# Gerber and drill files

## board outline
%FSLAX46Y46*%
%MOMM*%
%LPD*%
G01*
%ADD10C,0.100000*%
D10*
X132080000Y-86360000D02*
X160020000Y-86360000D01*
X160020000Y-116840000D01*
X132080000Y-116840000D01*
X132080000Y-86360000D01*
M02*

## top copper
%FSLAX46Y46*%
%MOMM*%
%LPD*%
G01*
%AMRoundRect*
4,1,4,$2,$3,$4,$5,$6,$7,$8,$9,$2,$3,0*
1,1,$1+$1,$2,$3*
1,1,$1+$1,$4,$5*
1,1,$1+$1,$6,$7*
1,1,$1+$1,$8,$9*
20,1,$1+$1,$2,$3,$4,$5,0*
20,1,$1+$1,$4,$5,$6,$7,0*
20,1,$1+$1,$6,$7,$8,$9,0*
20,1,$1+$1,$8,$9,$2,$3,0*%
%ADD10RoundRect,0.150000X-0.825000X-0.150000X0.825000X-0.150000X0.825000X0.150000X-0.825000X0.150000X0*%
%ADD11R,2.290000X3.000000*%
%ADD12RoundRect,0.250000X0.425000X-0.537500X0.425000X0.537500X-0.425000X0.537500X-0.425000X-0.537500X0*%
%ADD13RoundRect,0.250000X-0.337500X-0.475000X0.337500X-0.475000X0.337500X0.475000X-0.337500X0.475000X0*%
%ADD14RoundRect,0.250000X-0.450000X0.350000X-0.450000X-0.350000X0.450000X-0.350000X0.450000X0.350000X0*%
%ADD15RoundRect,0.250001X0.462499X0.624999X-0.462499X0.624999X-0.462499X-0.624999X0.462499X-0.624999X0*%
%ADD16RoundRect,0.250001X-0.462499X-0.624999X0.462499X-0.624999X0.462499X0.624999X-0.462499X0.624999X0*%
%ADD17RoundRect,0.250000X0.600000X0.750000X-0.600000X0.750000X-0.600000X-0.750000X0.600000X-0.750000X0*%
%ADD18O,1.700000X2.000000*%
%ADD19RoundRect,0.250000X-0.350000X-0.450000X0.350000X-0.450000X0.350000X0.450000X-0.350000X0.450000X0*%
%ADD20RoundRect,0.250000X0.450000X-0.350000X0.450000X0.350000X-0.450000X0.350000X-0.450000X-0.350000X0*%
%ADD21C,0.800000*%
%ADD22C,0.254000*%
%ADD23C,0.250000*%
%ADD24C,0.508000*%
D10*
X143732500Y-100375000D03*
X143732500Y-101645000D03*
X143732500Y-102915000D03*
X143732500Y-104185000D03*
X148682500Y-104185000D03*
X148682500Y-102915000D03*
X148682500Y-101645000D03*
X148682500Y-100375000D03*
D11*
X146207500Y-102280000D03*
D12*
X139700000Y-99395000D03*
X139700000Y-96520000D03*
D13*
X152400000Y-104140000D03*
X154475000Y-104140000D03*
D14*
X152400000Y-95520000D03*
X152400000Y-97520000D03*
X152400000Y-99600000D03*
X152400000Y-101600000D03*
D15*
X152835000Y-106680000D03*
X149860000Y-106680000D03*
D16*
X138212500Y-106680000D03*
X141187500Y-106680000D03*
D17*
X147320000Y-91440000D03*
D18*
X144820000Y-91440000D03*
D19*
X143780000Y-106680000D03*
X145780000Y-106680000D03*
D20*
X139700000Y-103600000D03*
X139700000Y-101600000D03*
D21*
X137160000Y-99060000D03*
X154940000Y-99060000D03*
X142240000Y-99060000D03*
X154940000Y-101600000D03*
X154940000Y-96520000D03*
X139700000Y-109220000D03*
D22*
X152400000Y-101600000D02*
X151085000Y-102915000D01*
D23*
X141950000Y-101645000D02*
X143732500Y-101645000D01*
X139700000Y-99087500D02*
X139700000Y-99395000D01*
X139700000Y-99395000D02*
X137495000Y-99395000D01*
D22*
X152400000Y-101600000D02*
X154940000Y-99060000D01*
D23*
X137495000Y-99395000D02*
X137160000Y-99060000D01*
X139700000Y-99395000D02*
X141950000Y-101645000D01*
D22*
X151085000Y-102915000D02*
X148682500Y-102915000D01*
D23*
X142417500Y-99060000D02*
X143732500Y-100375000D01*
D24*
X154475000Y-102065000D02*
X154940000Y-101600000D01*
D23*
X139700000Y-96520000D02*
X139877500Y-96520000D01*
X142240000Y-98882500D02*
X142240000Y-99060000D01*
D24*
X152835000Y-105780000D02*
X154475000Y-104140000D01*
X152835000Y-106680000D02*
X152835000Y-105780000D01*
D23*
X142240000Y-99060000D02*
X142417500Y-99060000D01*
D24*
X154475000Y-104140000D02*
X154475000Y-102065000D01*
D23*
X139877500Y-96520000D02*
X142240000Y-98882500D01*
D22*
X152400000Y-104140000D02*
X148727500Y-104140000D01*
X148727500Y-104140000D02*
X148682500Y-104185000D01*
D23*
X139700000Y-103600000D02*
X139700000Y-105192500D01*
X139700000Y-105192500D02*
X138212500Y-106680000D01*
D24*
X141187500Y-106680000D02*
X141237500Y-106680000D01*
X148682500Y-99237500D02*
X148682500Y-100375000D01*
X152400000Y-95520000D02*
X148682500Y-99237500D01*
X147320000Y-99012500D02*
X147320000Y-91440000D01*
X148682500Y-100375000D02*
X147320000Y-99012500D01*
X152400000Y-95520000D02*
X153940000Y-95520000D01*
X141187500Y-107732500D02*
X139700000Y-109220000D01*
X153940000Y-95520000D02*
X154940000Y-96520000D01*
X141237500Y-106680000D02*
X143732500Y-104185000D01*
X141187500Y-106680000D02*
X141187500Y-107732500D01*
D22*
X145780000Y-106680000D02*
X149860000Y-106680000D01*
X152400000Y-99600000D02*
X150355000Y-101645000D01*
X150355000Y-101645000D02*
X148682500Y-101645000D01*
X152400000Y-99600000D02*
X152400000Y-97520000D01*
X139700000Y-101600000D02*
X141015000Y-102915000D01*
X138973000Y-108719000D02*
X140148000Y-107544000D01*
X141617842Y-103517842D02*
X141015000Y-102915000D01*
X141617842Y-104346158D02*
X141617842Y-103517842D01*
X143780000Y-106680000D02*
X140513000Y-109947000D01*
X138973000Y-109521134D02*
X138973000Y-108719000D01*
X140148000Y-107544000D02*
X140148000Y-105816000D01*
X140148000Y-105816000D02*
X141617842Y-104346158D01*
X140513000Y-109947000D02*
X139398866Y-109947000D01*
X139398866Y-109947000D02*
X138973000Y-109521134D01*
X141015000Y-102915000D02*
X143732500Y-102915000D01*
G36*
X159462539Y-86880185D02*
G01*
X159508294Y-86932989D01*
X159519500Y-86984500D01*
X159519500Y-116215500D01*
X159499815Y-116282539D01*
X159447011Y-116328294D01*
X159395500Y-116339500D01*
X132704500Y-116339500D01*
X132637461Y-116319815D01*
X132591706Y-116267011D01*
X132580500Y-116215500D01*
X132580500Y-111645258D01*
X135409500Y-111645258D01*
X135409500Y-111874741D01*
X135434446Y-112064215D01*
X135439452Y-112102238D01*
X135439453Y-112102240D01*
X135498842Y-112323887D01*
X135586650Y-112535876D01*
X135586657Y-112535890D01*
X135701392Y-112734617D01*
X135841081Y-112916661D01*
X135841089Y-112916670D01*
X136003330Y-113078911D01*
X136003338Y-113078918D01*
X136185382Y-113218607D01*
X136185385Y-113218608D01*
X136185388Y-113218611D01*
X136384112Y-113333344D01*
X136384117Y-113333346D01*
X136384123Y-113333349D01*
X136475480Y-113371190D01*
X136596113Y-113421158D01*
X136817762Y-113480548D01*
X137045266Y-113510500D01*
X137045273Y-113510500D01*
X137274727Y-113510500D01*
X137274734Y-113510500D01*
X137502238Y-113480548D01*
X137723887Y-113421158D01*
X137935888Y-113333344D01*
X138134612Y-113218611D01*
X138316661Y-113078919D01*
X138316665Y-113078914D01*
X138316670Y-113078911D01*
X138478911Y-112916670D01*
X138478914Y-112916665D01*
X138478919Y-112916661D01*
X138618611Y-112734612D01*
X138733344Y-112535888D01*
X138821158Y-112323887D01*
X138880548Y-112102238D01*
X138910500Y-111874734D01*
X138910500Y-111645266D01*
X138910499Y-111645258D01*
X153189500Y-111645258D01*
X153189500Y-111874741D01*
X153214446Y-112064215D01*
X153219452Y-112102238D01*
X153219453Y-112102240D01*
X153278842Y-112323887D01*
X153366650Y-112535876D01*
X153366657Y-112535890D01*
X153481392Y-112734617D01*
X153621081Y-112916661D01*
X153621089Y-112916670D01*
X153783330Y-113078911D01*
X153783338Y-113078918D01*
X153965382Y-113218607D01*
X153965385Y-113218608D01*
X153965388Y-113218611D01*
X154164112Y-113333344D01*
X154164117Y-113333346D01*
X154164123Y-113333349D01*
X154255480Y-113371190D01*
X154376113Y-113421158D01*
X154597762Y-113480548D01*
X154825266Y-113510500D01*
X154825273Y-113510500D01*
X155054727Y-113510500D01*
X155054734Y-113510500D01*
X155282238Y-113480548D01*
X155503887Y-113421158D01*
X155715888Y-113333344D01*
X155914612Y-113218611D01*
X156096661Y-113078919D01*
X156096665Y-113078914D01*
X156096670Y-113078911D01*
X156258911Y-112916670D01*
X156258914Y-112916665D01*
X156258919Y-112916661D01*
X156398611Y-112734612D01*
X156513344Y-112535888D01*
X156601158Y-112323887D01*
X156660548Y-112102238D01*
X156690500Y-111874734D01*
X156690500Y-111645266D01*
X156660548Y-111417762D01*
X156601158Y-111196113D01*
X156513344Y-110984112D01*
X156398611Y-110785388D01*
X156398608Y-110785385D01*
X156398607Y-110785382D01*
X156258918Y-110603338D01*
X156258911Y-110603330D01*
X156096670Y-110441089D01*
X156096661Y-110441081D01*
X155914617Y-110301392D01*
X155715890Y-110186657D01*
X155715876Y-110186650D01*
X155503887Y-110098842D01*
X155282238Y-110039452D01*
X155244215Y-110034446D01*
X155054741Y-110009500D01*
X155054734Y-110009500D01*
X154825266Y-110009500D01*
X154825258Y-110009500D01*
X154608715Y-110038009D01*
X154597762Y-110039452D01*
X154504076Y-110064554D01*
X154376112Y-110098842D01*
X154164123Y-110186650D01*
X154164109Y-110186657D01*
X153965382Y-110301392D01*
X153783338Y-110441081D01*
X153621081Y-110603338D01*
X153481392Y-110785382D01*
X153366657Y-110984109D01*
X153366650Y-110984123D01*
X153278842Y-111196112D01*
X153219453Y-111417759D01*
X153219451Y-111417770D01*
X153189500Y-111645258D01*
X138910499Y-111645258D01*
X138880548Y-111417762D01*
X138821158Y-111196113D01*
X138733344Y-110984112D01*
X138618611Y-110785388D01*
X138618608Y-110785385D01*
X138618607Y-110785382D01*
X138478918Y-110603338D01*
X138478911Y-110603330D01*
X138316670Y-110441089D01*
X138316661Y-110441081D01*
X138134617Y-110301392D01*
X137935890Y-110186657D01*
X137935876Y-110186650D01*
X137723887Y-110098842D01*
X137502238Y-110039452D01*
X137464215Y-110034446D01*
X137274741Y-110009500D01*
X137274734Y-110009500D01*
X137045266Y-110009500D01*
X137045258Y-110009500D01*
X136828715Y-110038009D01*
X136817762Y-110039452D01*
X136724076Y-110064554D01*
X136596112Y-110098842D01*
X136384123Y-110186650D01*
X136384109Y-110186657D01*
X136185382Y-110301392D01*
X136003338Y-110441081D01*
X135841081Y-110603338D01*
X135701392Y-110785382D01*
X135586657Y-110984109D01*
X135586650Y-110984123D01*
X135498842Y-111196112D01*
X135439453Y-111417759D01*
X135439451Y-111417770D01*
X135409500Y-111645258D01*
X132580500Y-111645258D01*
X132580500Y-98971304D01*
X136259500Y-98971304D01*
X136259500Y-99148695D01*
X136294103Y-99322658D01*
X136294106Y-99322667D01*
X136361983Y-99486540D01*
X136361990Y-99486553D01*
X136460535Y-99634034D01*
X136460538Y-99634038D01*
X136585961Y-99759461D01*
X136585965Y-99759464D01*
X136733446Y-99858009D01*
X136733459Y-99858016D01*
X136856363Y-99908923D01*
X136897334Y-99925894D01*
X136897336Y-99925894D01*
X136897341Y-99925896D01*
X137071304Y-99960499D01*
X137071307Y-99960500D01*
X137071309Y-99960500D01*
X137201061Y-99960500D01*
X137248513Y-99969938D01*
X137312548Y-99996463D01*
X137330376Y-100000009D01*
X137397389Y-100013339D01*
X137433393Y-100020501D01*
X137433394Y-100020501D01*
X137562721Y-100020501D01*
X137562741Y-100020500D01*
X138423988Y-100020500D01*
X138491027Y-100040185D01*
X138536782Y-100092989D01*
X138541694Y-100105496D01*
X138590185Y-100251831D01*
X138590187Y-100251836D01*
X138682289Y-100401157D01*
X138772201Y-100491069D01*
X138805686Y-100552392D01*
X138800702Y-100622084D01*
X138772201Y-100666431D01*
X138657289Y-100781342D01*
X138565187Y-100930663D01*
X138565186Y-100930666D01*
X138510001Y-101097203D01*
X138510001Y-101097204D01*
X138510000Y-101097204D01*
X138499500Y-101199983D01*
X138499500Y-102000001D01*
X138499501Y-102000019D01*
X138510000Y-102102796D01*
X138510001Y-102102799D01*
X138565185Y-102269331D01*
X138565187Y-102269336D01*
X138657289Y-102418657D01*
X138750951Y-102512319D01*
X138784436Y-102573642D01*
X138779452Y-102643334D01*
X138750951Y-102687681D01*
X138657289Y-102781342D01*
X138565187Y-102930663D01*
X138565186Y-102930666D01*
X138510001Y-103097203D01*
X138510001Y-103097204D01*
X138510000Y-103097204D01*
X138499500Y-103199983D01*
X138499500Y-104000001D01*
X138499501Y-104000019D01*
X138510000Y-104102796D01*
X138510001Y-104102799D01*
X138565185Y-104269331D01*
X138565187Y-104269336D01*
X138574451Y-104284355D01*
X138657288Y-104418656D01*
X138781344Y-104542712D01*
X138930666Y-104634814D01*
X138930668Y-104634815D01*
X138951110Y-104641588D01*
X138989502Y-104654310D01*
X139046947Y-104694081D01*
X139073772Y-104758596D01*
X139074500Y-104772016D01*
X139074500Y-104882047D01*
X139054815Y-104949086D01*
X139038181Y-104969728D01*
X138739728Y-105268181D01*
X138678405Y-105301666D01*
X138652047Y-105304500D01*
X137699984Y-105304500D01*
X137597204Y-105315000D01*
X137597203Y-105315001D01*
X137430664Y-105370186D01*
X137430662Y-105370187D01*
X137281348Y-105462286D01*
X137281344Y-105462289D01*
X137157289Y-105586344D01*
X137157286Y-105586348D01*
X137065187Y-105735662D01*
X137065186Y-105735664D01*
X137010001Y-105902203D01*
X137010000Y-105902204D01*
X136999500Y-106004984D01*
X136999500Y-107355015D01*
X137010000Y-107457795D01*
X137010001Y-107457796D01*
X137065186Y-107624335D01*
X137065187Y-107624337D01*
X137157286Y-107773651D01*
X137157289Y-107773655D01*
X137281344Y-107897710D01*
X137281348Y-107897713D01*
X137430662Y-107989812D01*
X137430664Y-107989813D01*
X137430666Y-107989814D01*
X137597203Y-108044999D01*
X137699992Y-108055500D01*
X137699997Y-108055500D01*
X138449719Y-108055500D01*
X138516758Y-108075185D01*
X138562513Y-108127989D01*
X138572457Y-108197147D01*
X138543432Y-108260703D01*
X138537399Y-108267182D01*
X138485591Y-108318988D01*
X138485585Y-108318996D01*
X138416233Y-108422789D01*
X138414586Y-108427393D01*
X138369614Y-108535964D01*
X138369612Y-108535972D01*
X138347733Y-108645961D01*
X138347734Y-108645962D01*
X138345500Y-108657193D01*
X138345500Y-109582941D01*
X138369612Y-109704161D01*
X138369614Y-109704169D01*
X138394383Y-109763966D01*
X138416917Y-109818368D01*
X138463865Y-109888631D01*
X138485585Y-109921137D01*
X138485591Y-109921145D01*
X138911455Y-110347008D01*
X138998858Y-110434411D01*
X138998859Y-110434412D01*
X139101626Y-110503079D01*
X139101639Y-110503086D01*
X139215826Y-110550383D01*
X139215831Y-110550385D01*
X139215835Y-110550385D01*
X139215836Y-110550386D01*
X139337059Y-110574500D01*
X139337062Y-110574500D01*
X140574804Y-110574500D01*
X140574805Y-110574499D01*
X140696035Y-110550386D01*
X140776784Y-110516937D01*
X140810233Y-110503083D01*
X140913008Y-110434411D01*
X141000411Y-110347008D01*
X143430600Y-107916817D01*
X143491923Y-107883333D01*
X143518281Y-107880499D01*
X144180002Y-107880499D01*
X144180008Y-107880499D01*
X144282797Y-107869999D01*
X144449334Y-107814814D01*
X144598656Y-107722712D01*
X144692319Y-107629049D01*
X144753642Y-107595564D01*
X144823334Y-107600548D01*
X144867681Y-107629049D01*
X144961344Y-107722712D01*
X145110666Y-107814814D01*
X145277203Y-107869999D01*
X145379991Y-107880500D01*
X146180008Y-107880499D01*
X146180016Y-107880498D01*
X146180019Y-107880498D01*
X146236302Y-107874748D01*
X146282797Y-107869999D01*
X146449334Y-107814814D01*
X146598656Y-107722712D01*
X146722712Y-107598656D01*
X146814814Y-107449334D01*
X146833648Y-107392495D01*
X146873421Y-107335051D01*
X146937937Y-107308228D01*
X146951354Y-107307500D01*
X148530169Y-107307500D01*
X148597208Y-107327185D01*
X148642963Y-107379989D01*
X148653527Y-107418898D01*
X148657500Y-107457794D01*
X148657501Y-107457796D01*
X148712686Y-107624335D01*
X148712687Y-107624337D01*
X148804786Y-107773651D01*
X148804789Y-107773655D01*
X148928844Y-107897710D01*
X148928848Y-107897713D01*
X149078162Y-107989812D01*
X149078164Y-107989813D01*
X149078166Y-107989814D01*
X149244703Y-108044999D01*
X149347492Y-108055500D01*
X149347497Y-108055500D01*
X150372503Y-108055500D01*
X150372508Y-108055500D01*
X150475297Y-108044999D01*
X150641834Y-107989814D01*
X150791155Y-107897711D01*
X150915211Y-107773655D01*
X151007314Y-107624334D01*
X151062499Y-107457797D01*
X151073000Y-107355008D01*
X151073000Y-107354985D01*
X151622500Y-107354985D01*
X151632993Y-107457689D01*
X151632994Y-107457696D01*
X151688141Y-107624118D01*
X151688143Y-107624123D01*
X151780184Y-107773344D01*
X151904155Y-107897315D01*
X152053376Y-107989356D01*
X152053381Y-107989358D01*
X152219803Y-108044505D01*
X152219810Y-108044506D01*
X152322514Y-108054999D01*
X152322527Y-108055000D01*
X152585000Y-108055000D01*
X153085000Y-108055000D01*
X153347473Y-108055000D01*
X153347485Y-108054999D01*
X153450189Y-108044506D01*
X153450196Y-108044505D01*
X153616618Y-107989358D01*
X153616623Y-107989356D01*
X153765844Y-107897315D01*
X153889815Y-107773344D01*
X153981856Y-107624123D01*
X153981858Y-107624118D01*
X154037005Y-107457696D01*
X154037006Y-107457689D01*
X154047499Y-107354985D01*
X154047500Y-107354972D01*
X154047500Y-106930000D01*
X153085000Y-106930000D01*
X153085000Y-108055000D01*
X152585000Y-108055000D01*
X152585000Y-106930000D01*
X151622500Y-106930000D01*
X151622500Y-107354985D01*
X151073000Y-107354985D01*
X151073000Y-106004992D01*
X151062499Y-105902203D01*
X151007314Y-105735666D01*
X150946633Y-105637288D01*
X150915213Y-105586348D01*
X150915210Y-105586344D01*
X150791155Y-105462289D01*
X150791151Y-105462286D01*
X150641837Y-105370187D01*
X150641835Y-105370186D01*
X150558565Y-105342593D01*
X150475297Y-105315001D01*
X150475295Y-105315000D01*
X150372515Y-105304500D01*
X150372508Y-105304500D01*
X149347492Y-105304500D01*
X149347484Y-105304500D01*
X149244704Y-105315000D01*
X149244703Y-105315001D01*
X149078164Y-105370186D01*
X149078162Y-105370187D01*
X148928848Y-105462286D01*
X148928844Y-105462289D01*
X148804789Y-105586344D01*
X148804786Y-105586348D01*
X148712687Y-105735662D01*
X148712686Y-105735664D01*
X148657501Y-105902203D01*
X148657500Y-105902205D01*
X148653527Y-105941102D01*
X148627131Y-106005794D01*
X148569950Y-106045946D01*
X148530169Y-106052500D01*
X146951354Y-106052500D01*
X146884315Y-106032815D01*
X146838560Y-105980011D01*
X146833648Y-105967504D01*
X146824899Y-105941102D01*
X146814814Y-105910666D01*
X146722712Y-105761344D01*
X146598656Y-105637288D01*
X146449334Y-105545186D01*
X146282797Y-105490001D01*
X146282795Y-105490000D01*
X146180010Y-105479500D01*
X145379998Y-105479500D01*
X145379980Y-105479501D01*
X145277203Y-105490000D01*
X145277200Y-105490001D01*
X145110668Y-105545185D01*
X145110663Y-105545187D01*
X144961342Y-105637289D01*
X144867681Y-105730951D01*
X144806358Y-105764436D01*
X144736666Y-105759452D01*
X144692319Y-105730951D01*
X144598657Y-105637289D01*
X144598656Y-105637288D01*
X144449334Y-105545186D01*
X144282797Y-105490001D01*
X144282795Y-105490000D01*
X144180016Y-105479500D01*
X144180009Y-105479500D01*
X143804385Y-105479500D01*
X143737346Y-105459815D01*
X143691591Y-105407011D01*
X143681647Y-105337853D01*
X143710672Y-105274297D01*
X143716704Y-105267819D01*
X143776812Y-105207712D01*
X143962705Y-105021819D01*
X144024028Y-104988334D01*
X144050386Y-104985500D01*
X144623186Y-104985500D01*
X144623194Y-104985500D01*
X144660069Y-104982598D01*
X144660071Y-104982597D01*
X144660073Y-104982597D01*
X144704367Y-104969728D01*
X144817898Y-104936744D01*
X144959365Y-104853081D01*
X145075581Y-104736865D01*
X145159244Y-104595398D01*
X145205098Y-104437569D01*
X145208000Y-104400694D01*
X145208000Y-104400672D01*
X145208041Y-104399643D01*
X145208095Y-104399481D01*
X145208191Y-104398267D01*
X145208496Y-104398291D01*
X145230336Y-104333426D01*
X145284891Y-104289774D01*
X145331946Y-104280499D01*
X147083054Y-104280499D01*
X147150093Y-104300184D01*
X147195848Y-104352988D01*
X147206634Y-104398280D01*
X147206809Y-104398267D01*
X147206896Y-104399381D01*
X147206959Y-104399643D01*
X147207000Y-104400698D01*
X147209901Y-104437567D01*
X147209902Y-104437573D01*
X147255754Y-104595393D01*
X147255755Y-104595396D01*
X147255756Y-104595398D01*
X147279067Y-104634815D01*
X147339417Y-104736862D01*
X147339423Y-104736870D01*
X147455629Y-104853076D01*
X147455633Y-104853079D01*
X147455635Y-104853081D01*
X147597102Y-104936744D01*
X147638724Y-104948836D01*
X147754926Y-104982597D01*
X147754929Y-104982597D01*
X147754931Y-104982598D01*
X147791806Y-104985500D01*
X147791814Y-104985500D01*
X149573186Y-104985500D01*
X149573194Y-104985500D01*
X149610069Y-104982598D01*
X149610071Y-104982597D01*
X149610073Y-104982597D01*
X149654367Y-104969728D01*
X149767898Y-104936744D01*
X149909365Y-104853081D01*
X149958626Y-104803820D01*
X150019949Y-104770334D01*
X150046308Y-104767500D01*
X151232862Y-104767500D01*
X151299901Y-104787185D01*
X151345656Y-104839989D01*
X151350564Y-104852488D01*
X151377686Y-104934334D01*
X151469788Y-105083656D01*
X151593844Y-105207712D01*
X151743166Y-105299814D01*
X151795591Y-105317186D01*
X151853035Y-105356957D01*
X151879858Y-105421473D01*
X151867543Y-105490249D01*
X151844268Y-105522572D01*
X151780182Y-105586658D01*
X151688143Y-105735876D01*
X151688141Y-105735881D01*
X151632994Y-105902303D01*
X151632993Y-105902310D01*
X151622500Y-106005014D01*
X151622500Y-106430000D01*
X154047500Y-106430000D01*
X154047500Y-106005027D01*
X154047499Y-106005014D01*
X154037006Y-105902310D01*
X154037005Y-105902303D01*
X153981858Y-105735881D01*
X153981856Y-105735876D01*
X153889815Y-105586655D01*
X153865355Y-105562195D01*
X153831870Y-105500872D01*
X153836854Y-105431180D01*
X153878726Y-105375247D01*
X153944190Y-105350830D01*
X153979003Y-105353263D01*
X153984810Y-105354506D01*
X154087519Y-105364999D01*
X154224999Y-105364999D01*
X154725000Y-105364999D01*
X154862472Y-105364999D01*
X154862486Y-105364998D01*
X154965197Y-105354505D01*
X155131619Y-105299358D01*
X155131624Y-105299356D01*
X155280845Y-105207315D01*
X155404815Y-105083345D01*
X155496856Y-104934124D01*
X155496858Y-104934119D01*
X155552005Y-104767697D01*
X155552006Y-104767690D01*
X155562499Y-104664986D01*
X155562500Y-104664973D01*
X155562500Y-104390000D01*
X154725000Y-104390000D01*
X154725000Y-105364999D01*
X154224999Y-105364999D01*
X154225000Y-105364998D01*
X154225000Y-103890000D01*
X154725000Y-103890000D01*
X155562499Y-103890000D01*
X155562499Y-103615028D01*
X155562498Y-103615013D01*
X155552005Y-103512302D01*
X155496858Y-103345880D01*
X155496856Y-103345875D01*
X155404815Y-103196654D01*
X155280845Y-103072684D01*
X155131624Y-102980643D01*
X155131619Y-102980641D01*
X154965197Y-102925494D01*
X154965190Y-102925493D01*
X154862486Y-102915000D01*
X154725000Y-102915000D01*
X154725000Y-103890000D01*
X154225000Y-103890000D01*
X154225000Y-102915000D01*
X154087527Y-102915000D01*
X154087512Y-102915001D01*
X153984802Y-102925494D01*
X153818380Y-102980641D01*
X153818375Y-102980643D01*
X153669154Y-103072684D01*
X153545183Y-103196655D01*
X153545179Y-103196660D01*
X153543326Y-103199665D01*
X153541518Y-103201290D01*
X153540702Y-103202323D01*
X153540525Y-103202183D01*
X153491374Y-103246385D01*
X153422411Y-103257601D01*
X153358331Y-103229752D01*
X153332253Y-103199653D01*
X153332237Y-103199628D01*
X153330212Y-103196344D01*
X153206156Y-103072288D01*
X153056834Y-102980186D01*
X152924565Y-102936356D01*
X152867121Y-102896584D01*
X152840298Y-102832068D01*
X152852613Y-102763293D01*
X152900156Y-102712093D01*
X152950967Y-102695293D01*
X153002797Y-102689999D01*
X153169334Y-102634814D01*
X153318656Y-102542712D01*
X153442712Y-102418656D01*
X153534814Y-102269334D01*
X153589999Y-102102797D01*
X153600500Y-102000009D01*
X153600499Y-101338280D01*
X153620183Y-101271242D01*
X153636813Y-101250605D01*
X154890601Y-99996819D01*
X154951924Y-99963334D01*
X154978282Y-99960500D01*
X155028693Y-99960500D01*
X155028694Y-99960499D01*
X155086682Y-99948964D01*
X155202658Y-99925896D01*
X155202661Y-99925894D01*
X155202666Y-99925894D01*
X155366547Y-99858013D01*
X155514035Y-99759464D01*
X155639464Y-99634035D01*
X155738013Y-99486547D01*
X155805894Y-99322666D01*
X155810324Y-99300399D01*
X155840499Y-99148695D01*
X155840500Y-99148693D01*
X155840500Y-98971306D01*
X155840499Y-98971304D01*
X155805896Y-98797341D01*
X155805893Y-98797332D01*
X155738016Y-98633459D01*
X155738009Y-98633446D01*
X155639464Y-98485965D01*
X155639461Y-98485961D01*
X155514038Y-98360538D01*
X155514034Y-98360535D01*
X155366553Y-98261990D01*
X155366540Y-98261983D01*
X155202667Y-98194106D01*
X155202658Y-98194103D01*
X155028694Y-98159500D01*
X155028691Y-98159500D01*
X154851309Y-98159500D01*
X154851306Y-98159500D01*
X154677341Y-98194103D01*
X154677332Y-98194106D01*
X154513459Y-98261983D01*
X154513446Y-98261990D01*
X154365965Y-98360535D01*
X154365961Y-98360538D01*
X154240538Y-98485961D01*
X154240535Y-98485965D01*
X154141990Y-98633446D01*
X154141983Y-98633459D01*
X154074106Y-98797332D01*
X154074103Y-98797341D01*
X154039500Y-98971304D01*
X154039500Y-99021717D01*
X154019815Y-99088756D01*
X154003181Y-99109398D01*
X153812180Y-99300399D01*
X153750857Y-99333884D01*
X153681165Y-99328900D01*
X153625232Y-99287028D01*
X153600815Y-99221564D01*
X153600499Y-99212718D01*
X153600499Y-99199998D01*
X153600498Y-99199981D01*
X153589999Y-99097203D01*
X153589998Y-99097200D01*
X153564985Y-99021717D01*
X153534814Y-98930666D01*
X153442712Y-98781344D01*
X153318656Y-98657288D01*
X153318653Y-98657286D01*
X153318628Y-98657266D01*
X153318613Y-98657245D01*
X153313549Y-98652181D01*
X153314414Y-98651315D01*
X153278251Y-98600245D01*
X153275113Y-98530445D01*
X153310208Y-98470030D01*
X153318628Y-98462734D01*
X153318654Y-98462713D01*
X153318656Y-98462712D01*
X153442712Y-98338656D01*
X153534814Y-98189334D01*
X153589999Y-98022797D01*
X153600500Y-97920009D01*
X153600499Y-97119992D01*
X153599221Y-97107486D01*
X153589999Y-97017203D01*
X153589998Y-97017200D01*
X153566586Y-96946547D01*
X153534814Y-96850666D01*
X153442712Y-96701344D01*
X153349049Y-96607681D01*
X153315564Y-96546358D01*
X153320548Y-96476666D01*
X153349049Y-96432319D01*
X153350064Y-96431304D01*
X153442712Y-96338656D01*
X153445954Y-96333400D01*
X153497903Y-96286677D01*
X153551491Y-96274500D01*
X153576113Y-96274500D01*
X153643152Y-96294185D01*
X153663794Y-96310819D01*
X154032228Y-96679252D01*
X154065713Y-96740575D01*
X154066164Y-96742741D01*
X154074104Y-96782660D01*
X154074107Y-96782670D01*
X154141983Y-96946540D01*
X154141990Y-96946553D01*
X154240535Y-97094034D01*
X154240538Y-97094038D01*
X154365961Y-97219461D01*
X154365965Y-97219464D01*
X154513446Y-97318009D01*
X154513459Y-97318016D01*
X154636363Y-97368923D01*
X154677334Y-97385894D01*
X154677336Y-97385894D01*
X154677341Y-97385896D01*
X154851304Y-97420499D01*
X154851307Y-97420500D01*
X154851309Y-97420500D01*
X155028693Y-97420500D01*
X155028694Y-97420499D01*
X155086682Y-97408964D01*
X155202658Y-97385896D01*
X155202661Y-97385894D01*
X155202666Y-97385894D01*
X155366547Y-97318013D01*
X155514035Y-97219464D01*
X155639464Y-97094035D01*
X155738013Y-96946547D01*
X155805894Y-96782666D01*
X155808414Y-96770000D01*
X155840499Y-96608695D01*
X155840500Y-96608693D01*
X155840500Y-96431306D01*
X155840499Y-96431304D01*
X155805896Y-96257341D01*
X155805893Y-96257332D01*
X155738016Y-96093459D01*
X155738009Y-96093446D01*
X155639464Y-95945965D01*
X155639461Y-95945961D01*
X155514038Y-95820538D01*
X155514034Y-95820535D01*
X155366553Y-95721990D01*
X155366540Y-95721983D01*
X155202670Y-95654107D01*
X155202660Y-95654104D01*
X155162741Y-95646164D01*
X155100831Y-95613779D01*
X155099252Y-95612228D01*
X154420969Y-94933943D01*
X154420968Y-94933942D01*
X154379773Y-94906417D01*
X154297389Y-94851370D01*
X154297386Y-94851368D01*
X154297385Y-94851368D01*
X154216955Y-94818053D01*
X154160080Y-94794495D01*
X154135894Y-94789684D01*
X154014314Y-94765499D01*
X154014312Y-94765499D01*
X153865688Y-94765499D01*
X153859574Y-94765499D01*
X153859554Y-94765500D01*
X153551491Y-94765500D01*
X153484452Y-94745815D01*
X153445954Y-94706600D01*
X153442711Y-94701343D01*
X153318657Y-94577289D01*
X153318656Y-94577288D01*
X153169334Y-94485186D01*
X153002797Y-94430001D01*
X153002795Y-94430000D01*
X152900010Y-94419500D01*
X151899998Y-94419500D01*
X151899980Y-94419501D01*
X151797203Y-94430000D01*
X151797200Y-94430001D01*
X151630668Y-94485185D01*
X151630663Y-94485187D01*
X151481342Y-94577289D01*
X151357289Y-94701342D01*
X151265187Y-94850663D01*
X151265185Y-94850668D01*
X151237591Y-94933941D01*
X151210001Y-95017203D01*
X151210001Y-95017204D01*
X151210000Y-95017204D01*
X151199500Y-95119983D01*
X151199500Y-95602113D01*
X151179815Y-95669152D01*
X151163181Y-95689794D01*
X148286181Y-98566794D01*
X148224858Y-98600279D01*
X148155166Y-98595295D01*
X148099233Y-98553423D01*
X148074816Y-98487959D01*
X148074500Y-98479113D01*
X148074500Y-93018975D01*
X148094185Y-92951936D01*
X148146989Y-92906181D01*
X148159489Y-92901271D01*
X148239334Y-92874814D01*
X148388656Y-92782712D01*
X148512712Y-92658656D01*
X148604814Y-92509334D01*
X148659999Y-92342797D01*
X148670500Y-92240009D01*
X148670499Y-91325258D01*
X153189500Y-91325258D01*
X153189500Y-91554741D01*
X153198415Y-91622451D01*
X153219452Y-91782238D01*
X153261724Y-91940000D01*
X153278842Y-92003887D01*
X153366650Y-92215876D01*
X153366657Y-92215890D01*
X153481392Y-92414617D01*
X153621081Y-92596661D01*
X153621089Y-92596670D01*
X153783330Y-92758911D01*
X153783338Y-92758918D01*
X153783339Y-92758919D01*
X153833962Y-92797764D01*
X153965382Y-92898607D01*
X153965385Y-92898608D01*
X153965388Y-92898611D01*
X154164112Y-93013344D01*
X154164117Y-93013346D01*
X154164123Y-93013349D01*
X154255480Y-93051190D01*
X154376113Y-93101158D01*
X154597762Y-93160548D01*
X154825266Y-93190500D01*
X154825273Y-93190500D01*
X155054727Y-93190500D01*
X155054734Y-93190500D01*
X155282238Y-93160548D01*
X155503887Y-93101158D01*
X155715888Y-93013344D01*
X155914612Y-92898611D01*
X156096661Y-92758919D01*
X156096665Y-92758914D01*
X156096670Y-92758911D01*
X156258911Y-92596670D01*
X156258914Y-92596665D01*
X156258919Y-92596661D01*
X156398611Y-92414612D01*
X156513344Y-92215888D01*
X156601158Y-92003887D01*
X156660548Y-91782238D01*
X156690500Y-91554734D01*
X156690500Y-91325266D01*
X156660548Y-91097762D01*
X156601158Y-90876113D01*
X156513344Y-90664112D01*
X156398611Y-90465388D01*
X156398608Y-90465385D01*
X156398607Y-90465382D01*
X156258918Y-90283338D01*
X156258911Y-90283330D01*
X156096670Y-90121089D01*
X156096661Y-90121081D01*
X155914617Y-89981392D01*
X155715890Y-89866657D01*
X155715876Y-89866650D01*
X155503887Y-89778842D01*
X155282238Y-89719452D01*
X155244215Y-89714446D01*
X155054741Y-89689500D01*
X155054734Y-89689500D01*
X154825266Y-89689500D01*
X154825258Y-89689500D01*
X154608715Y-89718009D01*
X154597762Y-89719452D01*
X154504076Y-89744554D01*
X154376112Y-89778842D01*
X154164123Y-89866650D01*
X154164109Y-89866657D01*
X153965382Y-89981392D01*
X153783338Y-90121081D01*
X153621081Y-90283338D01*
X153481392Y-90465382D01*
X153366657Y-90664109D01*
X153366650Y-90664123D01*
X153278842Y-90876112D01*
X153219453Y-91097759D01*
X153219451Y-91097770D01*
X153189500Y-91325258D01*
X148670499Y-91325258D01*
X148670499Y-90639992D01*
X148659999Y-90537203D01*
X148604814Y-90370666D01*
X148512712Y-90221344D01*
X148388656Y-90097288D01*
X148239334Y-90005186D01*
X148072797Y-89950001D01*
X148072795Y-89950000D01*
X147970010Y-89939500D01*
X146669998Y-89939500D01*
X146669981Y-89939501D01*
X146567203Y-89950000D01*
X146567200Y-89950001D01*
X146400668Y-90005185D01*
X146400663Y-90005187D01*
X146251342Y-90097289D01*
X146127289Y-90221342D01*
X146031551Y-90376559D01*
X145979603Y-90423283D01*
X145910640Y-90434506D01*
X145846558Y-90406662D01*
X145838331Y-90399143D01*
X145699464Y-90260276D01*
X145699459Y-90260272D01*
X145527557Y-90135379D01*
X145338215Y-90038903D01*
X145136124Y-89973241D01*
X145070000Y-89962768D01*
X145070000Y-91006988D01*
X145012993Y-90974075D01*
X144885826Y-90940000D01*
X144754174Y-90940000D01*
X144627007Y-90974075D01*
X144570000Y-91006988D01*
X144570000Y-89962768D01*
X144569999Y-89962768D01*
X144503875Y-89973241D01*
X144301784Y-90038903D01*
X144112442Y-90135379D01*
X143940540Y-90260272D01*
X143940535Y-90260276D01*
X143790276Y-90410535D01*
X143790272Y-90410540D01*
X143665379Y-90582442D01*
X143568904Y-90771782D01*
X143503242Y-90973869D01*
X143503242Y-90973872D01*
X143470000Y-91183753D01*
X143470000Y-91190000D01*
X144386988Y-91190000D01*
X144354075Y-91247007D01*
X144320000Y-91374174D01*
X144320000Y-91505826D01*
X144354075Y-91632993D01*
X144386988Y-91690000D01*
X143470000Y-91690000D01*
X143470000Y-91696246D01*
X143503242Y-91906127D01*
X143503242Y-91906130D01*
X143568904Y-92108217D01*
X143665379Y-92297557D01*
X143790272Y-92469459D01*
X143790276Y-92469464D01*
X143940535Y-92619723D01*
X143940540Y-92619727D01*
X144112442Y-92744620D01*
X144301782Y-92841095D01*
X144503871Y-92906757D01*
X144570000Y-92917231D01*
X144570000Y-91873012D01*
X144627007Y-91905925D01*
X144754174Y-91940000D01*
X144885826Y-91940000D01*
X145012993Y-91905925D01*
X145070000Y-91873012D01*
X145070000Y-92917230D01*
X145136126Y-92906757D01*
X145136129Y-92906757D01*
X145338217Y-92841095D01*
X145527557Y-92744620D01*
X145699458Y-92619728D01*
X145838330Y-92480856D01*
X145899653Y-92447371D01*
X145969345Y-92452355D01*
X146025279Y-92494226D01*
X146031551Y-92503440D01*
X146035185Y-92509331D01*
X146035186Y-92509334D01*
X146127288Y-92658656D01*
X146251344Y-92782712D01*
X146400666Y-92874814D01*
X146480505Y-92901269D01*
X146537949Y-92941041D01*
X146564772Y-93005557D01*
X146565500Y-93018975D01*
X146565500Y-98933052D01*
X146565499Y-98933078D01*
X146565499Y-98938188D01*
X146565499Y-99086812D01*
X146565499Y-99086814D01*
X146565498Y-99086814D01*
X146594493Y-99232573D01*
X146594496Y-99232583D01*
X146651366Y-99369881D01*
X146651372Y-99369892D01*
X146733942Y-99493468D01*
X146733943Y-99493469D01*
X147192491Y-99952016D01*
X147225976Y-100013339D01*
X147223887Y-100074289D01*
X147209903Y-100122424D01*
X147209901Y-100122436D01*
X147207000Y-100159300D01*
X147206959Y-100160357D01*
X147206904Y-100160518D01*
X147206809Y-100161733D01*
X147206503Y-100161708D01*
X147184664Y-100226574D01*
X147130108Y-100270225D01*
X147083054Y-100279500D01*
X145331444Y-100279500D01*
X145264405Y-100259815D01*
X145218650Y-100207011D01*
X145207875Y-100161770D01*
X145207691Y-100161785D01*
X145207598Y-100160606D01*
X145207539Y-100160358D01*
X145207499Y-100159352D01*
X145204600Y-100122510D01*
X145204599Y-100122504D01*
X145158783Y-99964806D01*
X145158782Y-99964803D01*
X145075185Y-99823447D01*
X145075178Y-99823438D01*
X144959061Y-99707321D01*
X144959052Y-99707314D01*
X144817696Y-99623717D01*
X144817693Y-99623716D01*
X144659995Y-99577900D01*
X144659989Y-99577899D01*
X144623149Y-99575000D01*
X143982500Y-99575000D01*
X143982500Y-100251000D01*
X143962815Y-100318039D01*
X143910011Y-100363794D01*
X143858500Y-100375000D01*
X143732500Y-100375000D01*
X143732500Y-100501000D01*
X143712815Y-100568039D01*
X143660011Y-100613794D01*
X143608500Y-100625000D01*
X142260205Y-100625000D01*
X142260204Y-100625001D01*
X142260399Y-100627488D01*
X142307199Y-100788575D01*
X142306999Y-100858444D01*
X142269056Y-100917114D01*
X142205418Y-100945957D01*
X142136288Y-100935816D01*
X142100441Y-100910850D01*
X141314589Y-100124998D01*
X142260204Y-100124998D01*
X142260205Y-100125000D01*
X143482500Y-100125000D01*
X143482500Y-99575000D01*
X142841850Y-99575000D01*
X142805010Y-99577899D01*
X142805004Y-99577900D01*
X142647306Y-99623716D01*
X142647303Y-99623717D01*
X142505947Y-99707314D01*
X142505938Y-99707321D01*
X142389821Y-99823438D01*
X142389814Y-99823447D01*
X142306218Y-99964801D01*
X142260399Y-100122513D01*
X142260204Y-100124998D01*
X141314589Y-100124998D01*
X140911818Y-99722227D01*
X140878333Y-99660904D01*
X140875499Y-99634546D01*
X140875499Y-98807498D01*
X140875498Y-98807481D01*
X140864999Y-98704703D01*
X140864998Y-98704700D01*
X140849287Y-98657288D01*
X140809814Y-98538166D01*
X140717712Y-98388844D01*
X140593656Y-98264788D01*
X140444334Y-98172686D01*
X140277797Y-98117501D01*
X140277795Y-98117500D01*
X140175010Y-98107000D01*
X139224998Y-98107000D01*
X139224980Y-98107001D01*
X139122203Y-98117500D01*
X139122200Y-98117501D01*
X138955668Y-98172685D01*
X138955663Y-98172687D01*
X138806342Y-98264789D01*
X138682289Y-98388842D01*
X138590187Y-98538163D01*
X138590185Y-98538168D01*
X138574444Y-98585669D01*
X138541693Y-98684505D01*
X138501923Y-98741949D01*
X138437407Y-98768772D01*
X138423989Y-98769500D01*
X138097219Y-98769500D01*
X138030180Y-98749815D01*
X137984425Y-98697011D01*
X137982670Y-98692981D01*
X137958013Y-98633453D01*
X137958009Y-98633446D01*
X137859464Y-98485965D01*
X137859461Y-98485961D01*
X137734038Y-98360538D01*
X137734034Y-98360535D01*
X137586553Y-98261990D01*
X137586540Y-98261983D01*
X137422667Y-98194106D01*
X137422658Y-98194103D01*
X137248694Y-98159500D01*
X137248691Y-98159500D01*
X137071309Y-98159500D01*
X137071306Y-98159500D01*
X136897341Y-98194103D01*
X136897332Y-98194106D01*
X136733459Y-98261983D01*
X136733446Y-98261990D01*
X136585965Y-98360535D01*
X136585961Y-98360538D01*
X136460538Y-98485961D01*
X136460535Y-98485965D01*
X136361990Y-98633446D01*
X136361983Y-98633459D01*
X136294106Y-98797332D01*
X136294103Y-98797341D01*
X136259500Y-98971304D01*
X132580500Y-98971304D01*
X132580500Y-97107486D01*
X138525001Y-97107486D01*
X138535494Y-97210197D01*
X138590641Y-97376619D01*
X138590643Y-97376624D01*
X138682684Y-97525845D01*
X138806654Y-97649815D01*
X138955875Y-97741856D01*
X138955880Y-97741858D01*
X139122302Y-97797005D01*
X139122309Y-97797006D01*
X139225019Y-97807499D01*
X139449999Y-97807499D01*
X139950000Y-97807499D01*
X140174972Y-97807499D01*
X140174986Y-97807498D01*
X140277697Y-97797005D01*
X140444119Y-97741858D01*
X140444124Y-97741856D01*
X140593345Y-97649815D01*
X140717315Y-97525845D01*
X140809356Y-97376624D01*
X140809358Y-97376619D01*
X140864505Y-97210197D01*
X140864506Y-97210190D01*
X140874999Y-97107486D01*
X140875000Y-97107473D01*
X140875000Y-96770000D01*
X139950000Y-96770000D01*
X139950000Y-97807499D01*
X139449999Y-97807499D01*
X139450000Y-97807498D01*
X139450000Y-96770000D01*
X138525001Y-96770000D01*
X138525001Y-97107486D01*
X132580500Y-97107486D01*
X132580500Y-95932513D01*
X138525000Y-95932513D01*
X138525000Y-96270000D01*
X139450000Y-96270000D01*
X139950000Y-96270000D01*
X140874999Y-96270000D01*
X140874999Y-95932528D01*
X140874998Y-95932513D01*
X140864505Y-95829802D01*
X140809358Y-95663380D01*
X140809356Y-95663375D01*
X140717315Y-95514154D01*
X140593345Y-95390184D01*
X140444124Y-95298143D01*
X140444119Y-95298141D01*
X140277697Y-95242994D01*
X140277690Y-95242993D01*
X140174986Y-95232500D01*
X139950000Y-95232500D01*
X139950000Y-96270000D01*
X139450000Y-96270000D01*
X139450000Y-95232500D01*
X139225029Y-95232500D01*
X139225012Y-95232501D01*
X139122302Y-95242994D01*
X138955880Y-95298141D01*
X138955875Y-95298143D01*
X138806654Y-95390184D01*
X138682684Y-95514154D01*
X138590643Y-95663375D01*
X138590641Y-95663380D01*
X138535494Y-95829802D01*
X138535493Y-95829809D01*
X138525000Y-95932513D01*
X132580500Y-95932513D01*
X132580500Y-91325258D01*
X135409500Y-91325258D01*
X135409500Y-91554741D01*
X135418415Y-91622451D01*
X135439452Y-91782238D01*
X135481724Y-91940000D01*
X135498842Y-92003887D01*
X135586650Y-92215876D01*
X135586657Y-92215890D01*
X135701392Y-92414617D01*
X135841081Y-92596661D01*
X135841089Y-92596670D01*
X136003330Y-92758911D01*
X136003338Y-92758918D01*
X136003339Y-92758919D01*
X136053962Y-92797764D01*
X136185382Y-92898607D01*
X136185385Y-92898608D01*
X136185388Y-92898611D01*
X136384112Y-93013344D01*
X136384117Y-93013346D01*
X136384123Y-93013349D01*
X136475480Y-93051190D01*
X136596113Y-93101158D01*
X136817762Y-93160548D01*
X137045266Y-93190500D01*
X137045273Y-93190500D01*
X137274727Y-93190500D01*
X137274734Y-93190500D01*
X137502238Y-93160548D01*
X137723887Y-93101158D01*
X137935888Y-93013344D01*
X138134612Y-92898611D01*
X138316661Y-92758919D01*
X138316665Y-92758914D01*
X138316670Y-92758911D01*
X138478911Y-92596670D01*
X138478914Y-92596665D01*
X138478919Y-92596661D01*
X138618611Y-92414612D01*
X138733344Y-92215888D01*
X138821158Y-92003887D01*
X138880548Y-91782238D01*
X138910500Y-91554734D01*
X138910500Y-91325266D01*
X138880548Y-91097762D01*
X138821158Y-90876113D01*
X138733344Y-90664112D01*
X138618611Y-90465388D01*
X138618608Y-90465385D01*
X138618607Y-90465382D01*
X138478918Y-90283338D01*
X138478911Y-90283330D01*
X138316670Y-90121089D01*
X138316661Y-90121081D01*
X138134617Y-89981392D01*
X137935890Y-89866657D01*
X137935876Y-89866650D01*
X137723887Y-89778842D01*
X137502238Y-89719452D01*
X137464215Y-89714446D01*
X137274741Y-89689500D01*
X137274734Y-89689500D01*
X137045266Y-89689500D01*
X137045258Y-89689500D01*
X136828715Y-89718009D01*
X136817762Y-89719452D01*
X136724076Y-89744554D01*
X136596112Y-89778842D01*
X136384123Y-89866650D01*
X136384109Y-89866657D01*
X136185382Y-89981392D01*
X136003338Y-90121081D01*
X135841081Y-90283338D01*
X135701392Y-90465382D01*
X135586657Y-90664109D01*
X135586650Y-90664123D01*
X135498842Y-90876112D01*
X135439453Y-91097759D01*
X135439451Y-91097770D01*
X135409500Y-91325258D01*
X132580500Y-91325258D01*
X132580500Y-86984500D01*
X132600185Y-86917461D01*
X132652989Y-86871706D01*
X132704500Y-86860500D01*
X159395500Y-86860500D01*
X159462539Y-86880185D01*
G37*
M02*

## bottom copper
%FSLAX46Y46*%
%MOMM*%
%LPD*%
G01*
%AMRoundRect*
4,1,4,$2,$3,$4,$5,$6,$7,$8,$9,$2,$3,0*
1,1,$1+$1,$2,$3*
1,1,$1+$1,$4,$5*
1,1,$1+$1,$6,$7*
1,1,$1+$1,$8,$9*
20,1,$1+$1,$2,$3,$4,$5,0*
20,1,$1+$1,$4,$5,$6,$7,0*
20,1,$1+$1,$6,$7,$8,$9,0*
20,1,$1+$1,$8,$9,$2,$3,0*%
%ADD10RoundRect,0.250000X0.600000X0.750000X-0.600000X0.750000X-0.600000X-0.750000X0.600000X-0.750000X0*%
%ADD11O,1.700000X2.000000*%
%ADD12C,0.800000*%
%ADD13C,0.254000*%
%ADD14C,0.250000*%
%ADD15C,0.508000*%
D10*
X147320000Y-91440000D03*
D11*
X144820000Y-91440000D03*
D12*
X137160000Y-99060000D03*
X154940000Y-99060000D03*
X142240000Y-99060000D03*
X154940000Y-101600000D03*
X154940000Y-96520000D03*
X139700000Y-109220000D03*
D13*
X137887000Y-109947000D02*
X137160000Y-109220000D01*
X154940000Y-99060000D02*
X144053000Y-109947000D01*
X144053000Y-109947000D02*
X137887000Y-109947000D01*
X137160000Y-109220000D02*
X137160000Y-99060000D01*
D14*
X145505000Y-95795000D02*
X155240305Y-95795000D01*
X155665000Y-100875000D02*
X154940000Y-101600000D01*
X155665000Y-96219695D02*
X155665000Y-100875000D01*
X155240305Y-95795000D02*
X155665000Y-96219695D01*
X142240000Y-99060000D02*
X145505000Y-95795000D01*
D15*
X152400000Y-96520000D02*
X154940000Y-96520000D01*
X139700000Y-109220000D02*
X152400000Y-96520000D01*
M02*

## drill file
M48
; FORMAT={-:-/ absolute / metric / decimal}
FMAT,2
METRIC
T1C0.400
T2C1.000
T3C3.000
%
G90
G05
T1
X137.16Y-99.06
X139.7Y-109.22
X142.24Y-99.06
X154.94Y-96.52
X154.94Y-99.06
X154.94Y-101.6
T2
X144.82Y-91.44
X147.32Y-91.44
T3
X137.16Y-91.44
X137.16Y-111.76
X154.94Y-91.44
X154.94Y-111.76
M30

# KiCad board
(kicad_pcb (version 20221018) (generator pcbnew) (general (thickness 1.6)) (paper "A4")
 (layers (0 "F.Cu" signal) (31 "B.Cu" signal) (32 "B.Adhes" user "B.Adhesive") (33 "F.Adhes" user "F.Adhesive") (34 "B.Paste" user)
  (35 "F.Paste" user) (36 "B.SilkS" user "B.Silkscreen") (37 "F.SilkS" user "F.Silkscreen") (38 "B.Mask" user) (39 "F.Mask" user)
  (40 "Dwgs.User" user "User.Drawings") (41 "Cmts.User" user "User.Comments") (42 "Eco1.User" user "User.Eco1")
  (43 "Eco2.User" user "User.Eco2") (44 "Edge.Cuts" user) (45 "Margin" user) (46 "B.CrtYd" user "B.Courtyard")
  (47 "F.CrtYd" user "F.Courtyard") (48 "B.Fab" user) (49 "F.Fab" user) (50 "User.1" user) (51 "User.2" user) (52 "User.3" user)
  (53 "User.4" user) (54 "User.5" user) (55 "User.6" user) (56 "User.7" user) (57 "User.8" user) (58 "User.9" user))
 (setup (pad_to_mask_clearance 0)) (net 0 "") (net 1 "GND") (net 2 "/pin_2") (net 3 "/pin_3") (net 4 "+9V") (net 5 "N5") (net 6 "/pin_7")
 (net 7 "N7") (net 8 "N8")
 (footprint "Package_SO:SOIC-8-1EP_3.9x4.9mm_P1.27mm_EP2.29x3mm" (layer "F.Cu") (at 146.2075 102.28)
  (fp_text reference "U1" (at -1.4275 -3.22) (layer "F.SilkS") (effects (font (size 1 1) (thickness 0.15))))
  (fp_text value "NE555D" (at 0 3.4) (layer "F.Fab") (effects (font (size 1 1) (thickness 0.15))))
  (pad "" smd roundrect (at -0.57 -0.75) (size 0.92 1.21) (layers "F.Paste") (roundrect_rratio 0.25))
  (pad "" smd roundrect (at -0.57 0.75) (size 0.92 1.21) (layers "F.Paste") (roundrect_rratio 0.25))
  (pad "" smd roundrect (at 0.57 -0.75) (size 0.92 1.21) (layers "F.Paste") (roundrect_rratio 0.25))
  (pad "" smd roundrect (at 0.57 0.75) (size 0.92 1.21) (layers "F.Paste") (roundrect_rratio 0.25))
  (pad "1" smd roundrect (at -2.475 -1.905) (size 1.95 0.6) (layers "F.Cu" "F.Paste" "F.Mask") (roundrect_rratio 0.25) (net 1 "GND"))
  (pad "2" smd roundrect (at -2.475 -0.635) (size 1.95 0.6) (layers "F.Cu" "F.Paste" "F.Mask") (roundrect_rratio 0.25) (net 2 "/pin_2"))
  (pad "3" smd roundrect (at -2.475 0.635) (size 1.95 0.6) (layers "F.Cu" "F.Paste" "F.Mask") (roundrect_rratio 0.25) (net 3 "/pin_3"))
  (pad "4" smd roundrect (at -2.475 1.905) (size 1.95 0.6) (layers "F.Cu" "F.Paste" "F.Mask") (roundrect_rratio 0.25) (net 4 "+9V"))
  (pad "5" smd roundrect (at 2.475 1.905) (size 1.95 0.6) (layers "F.Cu" "F.Paste" "F.Mask") (roundrect_rratio 0.25) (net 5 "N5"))
  (pad "6" smd roundrect (at 2.475 0.635) (size 1.95 0.6) (layers "F.Cu" "F.Paste" "F.Mask") (roundrect_rratio 0.25) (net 2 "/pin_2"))
  (pad "7" smd roundrect (at 2.475 -0.635) (size 1.95 0.6) (layers "F.Cu" "F.Paste" "F.Mask") (roundrect_rratio 0.25) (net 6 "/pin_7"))
  (pad "8" smd roundrect (at 2.475 -1.905) (size 1.95 0.6) (layers "F.Cu" "F.Paste" "F.Mask") (roundrect_rratio 0.25) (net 4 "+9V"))
  (pad "9" smd rect (at 0 0) (size 2.29 3) (layers "F.Cu" "F.Mask")))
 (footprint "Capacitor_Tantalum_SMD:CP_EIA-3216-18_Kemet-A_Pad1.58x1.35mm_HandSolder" (layer "F.Cu") (at 139.7 97.9575 90)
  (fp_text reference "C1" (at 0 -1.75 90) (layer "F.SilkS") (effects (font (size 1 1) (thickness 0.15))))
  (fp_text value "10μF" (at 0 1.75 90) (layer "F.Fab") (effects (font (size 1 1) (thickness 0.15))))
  (pad "1" smd roundrect (at -1.4375 0 90) (size 1.575 1.35) (layers "F.Cu" "F.Paste" "F.Mask") (roundrect_rratio 0.185185) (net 2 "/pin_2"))
  (pad "2" smd roundrect (at 1.4375 0 90) (size 1.575 1.35) (layers "F.Cu" "F.Paste" "F.Mask") (roundrect_rratio 0.185185) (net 1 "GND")))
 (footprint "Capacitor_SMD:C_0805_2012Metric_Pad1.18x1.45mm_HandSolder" (layer "F.Cu") (at 153.4375 104.14)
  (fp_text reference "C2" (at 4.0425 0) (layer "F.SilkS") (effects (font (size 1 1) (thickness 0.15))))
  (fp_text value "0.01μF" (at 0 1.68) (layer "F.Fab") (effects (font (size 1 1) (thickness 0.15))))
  (pad "1" smd roundrect (at -1.0375 0) (size 1.175 1.45) (layers "F.Cu" "F.Paste" "F.Mask") (roundrect_rratio 0.212766) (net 5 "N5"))
  (pad "2" smd roundrect (at 1.0375 0) (size 1.175 1.45) (layers "F.Cu" "F.Paste" "F.Mask") (roundrect_rratio 0.212766) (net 1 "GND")))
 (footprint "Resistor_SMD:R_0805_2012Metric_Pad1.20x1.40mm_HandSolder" (layer "F.Cu") (at 152.4 96.52 -90)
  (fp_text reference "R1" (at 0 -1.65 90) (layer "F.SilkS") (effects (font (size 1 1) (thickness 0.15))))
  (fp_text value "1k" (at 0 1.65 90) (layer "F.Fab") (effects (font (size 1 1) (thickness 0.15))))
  (pad "1" smd roundrect (at -1 0 270) (size 1.2 1.4) (layers "F.Cu" "F.Paste" "F.Mask") (roundrect_rratio 0.208333) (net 4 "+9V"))
  (pad "2" smd roundrect (at 1 0 270) (size 1.2 1.4) (layers "F.Cu" "F.Paste" "F.Mask") (roundrect_rratio 0.208333) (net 6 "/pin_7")))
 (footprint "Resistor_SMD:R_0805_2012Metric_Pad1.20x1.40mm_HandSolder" (layer "F.Cu") (at 152.4 100.6 -90)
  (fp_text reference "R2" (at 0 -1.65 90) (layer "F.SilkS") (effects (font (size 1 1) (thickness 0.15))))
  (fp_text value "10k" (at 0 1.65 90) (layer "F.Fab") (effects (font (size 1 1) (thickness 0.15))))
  (pad "1" smd roundrect (at -1 0 270) (size 1.2 1.4) (layers "F.Cu" "F.Paste" "F.Mask") (roundrect_rratio 0.208333) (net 6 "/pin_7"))
  (pad "2" smd roundrect (at 1 0 270) (size 1.2 1.4) (layers "F.Cu" "F.Paste" "F.Mask") (roundrect_rratio 0.208333) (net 2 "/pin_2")))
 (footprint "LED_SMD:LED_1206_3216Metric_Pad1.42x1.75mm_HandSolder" (layer "F.Cu") (at 151.3475 106.68 180)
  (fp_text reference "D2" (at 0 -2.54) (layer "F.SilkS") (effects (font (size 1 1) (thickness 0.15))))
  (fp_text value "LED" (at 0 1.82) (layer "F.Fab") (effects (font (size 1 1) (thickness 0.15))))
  (pad "1" smd roundrect (at -1.4875 0 180) (size 1.425 1.75) (layers "F.Cu" "F.Paste" "F.Mask") (roundrect_rratio 0.175439) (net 1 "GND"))
  (pad "2" smd roundrect (at 1.4875 0 180) (size 1.425 1.75) (layers "F.Cu" "F.Paste" "F.Mask") (roundrect_rratio 0.175439) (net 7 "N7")))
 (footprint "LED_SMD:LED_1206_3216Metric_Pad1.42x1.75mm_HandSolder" (layer "F.Cu") (at 139.7 106.68)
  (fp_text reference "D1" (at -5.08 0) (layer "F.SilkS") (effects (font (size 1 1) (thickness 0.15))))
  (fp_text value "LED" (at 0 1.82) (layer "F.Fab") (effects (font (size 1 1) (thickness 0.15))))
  (pad "1" smd roundrect (at -1.4875 0) (size 1.425 1.75) (layers "F.Cu" "F.Paste" "F.Mask") (roundrect_rratio 0.175439) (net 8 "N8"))
  (pad "2" smd roundrect (at 1.4875 0) (size 1.425 1.75) (layers "F.Cu" "F.Paste" "F.Mask") (roundrect_rratio 0.175439) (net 4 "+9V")))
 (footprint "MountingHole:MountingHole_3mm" (layer "F.Cu") (at 154.94 91.44)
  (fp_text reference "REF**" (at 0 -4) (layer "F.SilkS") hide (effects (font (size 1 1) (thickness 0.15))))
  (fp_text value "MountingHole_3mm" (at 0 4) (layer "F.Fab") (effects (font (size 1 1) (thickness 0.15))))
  (pad "" np_thru_hole circle (at 0 0) (size 3 3) (drill 3) (layers "*.Cu" "*.Mask")))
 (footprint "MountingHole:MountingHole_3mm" (layer "F.Cu") (at 137.16 111.76)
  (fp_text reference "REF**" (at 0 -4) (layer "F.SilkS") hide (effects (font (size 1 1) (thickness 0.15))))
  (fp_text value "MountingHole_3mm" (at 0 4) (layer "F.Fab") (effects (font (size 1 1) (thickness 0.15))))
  (pad "" np_thru_hole circle (at 0 0) (size 3 3) (drill 3) (layers "*.Cu" "*.Mask")))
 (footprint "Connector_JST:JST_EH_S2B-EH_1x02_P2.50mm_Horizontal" (layer "F.Cu") (at 147.32 91.44 180)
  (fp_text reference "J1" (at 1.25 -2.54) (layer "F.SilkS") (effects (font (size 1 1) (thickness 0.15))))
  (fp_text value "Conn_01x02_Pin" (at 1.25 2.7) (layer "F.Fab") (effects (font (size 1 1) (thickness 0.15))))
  (pad "1" thru_hole roundrect (at 0 0 180) (size 1.7 2) (drill 1) (layers "*.Cu" "*.Mask") (roundrect_rratio 0.147059) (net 4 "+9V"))
  (pad "2" thru_hole oval (at 2.5 0 180) (size 1.7 2) (drill 1) (layers "*.Cu" "*.Mask") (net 1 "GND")))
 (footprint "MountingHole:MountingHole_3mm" (layer "F.Cu") (at 137.16 91.44)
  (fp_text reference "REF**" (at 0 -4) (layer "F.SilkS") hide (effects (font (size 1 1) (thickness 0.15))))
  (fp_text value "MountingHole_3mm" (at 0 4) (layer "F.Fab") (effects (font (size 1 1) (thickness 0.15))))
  (pad "" np_thru_hole circle (at 0 0) (size 3 3) (drill 3) (layers "*.Cu" "*.Mask")))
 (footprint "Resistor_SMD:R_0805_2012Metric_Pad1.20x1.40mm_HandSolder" (layer "F.Cu") (at 144.78 106.68)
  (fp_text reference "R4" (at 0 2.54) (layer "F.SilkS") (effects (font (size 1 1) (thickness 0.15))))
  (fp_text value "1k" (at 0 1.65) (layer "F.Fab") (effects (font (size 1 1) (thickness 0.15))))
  (pad "1" smd roundrect (at -1 0) (size 1.2 1.4) (layers "F.Cu" "F.Paste" "F.Mask") (roundrect_rratio 0.208333) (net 3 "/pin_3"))
  (pad "2" smd roundrect (at 1 0) (size 1.2 1.4) (layers "F.Cu" "F.Paste" "F.Mask") (roundrect_rratio 0.208333) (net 7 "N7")))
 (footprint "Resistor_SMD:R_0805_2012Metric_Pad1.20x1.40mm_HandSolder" (layer "F.Cu") (at 139.7 102.6 90)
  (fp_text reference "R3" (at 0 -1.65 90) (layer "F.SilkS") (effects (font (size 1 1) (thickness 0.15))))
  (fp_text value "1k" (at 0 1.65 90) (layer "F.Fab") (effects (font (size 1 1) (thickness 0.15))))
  (pad "1" smd roundrect (at -1 0 90) (size 1.2 1.4) (layers "F.Cu" "F.Paste" "F.Mask") (roundrect_rratio 0.208333) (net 8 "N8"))
  (pad "2" smd roundrect (at 1 0 90) (size 1.2 1.4) (layers "F.Cu" "F.Paste" "F.Mask") (roundrect_rratio 0.208333) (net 3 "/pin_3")))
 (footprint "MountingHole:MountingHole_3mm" (layer "F.Cu") (at 154.94 111.76)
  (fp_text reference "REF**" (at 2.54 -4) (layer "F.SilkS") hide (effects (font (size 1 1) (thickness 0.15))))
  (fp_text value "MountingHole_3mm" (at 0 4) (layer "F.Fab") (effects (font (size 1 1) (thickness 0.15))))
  (pad "" np_thru_hole circle (at 0 0) (size 3 3) (drill 3) (layers "*.Cu" "*.Mask")))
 (gr_rect (start 132.08 86.36) (end 160.02 116.84) (stroke (width 0.1) (type default)) (fill none) (layer "Edge.Cuts"))
 (segment (start 152.4 101.6) (end 151.085 102.915) (width 0.254) (layer "F.Cu") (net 2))
 (segment (start 141.95 101.645) (end 143.7325 101.645) (width 0.25) (layer "F.Cu") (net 2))
 (segment (start 139.7 99.0875) (end 139.7 99.395) (width 0.25) (layer "F.Cu") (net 2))
 (segment (start 139.7 99.395) (end 137.495 99.395) (width 0.25) (layer "F.Cu") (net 2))
 (segment (start 152.4 101.6) (end 154.94 99.06) (width 0.254) (layer "F.Cu") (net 2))
 (segment (start 137.495 99.395) (end 137.16 99.06) (width 0.25) (layer "F.Cu") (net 2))
 (segment (start 139.7 99.395) (end 141.95 101.645) (width 0.25) (layer "F.Cu") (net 2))
 (segment (start 151.085 102.915) (end 148.6825 102.915) (width 0.254) (layer "F.Cu") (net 2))
 (via (at 137.16 99.06) (size 0.8) (drill 0.4) (layers "F.Cu" "B.Cu") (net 2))
 (via (at 154.94 99.06) (size 0.8) (drill 0.4) (layers "F.Cu" "B.Cu") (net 2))
 (segment (start 137.887 109.947) (end 137.16 109.22) (width 0.254) (layer "B.Cu") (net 2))
 (segment (start 154.94 99.06) (end 144.053 109.947) (width 0.254) (layer "B.Cu") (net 2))
 (segment (start 144.053 109.947) (end 137.887 109.947) (width 0.254) (layer "B.Cu") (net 2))
 (segment (start 137.16 109.22) (end 137.16 99.06) (width 0.254) (layer "B.Cu") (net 2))
 (segment (start 142.4175 99.06) (end 143.7325 100.375) (width 0.25) (layer "F.Cu") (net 1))
 (segment (start 154.475 102.065) (end 154.94 101.6) (width 0.508) (layer "F.Cu") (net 1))
 (segment (start 139.7 96.52) (end 139.8775 96.52) (width 0.25) (layer "F.Cu") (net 1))
 (segment (start 142.24 98.8825) (end 142.24 99.06) (width 0.25) (layer "F.Cu") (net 1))
 (segment (start 152.835 105.78) (end 154.475 104.14) (width 0.508) (layer "F.Cu") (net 1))
 (segment (start 152.835 106.68) (end 152.835 105.78) (width 0.508) (layer "F.Cu") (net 1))
 (segment (start 142.24 99.06) (end 142.4175 99.06) (width 0.25) (layer "F.Cu") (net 1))
 (segment (start 154.475 104.14) (end 154.475 102.065) (width 0.508) (layer "F.Cu") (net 1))
 (segment (start 139.8775 96.52) (end 142.24 98.8825) (width 0.25) (layer "F.Cu") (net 1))
 (via (at 142.24 99.06) (size 0.8) (drill 0.4) (layers "F.Cu" "B.Cu") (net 1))
 (via (at 154.94 101.6) (size 0.8) (drill 0.4) (layers "F.Cu" "B.Cu") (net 1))
 (segment (start 145.505 95.795) (end 155.240305 95.795) (width 0.25) (layer "B.Cu") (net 1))
 (segment (start 155.665 100.875) (end 154.94 101.6) (width 0.25) (layer "B.Cu") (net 1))
 (segment (start 155.665 96.219695) (end 155.665 100.875) (width 0.25) (layer "B.Cu") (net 1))
 (segment (start 155.240305 95.795) (end 155.665 96.219695) (width 0.25) (layer "B.Cu") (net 1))
 (segment (start 142.24 99.06) (end 145.505 95.795) (width 0.25) (layer "B.Cu") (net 1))
 (segment (start 152.4 104.14) (end 148.7275 104.14) (width 0.254) (layer "F.Cu") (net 5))
 (segment (start 148.7275 104.14) (end 148.6825 104.185) (width 0.254) (layer "F.Cu") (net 5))
 (segment (start 139.7 103.6) (end 139.7 105.1925) (width 0.25) (layer "F.Cu") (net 8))
 (segment (start 139.7 105.1925) (end 138.2125 106.68) (width 0.25) (layer "F.Cu") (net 8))
 (segment (start 141.1875 106.68) (end 141.2375 106.68) (width 0.508) (layer "F.Cu") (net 4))
 (segment (start 148.6825 99.2375) (end 148.6825 100.375) (width 0.508) (layer "F.Cu") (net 4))
 (segment (start 152.4 95.52) (end 148.6825 99.2375) (width 0.508) (layer "F.Cu") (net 4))
 (segment (start 147.32 99.0125) (end 147.32 91.44) (width 0.508) (layer "F.Cu") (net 4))
 (segment (start 148.6825 100.375) (end 147.32 99.0125) (width 0.508) (layer "F.Cu") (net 4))
 (segment (start 152.4 95.52) (end 153.94 95.52) (width 0.508) (layer "F.Cu") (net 4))
 (segment (start 141.1875 107.7325) (end 139.7 109.22) (width 0.508) (layer "F.Cu") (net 4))
 (segment (start 153.94 95.52) (end 154.94 96.52) (width 0.508) (layer "F.Cu") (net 4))
 (segment (start 141.2375 106.68) (end 143.7325 104.185) (width 0.508) (layer "F.Cu") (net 4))
 (segment (start 141.1875 106.68) (end 141.1875 107.7325) (width 0.508) (layer "F.Cu") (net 4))
 (via (at 154.94 96.52) (size 0.8) (drill 0.4) (layers "F.Cu" "B.Cu") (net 4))
 (via (at 139.7 109.22) (size 0.8) (drill 0.4) (layers "F.Cu" "B.Cu") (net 4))
 (segment (start 152.4 96.52) (end 154.94 96.52) (width 0.508) (layer "B.Cu") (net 4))
 (segment (start 139.7 109.22) (end 152.4 96.52) (width 0.508) (layer "B.Cu") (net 4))
 (segment (start 145.78 106.68) (end 149.86 106.68) (width 0.254) (layer "F.Cu") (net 7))
 (segment (start 152.4 99.6) (end 150.355 101.645) (width 0.254) (layer "F.Cu") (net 6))
 (segment (start 150.355 101.645) (end 148.6825 101.645) (width 0.254) (layer "F.Cu") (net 6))
 (segment (start 152.4 99.6) (end 152.4 97.52) (width 0.254) (layer "F.Cu") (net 6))
 (segment (start 139.7 101.6) (end 141.015 102.915) (width 0.254) (layer "F.Cu") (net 3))
 (segment (start 138.973 108.719) (end 140.148 107.544) (width 0.254) (layer "F.Cu") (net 3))
 (segment (start 141.617842 103.517842) (end 141.015 102.915) (width 0.254) (layer "F.Cu") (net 3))
 (segment (start 141.617842 104.346158) (end 141.617842 103.517842) (width 0.254) (layer "F.Cu") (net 3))
 (segment (start 143.78 106.68) (end 140.513 109.947) (width 0.254) (layer "F.Cu") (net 3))
 (segment (start 138.973 109.521134) (end 138.973 108.719) (width 0.254) (layer "F.Cu") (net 3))
 (segment (start 140.148 107.544) (end 140.148 105.816) (width 0.254) (layer "F.Cu") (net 3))
 (segment (start 140.148 105.816) (end 141.617842 104.346158) (width 0.254) (layer "F.Cu") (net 3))
 (segment (start 140.513 109.947) (end 139.398866 109.947) (width 0.254) (layer "F.Cu") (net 3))
 (segment (start 139.398866 109.947) (end 138.973 109.521134) (width 0.254) (layer "F.Cu") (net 3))
 (segment (start 141.015 102.915) (end 143.7325 102.915) (width 0.254) (layer "F.Cu") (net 3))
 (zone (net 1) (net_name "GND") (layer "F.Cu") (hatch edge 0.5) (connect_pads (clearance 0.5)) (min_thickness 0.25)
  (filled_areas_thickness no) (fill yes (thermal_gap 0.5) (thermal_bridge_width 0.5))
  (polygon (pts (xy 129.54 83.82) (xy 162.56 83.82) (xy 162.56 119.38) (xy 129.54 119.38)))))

